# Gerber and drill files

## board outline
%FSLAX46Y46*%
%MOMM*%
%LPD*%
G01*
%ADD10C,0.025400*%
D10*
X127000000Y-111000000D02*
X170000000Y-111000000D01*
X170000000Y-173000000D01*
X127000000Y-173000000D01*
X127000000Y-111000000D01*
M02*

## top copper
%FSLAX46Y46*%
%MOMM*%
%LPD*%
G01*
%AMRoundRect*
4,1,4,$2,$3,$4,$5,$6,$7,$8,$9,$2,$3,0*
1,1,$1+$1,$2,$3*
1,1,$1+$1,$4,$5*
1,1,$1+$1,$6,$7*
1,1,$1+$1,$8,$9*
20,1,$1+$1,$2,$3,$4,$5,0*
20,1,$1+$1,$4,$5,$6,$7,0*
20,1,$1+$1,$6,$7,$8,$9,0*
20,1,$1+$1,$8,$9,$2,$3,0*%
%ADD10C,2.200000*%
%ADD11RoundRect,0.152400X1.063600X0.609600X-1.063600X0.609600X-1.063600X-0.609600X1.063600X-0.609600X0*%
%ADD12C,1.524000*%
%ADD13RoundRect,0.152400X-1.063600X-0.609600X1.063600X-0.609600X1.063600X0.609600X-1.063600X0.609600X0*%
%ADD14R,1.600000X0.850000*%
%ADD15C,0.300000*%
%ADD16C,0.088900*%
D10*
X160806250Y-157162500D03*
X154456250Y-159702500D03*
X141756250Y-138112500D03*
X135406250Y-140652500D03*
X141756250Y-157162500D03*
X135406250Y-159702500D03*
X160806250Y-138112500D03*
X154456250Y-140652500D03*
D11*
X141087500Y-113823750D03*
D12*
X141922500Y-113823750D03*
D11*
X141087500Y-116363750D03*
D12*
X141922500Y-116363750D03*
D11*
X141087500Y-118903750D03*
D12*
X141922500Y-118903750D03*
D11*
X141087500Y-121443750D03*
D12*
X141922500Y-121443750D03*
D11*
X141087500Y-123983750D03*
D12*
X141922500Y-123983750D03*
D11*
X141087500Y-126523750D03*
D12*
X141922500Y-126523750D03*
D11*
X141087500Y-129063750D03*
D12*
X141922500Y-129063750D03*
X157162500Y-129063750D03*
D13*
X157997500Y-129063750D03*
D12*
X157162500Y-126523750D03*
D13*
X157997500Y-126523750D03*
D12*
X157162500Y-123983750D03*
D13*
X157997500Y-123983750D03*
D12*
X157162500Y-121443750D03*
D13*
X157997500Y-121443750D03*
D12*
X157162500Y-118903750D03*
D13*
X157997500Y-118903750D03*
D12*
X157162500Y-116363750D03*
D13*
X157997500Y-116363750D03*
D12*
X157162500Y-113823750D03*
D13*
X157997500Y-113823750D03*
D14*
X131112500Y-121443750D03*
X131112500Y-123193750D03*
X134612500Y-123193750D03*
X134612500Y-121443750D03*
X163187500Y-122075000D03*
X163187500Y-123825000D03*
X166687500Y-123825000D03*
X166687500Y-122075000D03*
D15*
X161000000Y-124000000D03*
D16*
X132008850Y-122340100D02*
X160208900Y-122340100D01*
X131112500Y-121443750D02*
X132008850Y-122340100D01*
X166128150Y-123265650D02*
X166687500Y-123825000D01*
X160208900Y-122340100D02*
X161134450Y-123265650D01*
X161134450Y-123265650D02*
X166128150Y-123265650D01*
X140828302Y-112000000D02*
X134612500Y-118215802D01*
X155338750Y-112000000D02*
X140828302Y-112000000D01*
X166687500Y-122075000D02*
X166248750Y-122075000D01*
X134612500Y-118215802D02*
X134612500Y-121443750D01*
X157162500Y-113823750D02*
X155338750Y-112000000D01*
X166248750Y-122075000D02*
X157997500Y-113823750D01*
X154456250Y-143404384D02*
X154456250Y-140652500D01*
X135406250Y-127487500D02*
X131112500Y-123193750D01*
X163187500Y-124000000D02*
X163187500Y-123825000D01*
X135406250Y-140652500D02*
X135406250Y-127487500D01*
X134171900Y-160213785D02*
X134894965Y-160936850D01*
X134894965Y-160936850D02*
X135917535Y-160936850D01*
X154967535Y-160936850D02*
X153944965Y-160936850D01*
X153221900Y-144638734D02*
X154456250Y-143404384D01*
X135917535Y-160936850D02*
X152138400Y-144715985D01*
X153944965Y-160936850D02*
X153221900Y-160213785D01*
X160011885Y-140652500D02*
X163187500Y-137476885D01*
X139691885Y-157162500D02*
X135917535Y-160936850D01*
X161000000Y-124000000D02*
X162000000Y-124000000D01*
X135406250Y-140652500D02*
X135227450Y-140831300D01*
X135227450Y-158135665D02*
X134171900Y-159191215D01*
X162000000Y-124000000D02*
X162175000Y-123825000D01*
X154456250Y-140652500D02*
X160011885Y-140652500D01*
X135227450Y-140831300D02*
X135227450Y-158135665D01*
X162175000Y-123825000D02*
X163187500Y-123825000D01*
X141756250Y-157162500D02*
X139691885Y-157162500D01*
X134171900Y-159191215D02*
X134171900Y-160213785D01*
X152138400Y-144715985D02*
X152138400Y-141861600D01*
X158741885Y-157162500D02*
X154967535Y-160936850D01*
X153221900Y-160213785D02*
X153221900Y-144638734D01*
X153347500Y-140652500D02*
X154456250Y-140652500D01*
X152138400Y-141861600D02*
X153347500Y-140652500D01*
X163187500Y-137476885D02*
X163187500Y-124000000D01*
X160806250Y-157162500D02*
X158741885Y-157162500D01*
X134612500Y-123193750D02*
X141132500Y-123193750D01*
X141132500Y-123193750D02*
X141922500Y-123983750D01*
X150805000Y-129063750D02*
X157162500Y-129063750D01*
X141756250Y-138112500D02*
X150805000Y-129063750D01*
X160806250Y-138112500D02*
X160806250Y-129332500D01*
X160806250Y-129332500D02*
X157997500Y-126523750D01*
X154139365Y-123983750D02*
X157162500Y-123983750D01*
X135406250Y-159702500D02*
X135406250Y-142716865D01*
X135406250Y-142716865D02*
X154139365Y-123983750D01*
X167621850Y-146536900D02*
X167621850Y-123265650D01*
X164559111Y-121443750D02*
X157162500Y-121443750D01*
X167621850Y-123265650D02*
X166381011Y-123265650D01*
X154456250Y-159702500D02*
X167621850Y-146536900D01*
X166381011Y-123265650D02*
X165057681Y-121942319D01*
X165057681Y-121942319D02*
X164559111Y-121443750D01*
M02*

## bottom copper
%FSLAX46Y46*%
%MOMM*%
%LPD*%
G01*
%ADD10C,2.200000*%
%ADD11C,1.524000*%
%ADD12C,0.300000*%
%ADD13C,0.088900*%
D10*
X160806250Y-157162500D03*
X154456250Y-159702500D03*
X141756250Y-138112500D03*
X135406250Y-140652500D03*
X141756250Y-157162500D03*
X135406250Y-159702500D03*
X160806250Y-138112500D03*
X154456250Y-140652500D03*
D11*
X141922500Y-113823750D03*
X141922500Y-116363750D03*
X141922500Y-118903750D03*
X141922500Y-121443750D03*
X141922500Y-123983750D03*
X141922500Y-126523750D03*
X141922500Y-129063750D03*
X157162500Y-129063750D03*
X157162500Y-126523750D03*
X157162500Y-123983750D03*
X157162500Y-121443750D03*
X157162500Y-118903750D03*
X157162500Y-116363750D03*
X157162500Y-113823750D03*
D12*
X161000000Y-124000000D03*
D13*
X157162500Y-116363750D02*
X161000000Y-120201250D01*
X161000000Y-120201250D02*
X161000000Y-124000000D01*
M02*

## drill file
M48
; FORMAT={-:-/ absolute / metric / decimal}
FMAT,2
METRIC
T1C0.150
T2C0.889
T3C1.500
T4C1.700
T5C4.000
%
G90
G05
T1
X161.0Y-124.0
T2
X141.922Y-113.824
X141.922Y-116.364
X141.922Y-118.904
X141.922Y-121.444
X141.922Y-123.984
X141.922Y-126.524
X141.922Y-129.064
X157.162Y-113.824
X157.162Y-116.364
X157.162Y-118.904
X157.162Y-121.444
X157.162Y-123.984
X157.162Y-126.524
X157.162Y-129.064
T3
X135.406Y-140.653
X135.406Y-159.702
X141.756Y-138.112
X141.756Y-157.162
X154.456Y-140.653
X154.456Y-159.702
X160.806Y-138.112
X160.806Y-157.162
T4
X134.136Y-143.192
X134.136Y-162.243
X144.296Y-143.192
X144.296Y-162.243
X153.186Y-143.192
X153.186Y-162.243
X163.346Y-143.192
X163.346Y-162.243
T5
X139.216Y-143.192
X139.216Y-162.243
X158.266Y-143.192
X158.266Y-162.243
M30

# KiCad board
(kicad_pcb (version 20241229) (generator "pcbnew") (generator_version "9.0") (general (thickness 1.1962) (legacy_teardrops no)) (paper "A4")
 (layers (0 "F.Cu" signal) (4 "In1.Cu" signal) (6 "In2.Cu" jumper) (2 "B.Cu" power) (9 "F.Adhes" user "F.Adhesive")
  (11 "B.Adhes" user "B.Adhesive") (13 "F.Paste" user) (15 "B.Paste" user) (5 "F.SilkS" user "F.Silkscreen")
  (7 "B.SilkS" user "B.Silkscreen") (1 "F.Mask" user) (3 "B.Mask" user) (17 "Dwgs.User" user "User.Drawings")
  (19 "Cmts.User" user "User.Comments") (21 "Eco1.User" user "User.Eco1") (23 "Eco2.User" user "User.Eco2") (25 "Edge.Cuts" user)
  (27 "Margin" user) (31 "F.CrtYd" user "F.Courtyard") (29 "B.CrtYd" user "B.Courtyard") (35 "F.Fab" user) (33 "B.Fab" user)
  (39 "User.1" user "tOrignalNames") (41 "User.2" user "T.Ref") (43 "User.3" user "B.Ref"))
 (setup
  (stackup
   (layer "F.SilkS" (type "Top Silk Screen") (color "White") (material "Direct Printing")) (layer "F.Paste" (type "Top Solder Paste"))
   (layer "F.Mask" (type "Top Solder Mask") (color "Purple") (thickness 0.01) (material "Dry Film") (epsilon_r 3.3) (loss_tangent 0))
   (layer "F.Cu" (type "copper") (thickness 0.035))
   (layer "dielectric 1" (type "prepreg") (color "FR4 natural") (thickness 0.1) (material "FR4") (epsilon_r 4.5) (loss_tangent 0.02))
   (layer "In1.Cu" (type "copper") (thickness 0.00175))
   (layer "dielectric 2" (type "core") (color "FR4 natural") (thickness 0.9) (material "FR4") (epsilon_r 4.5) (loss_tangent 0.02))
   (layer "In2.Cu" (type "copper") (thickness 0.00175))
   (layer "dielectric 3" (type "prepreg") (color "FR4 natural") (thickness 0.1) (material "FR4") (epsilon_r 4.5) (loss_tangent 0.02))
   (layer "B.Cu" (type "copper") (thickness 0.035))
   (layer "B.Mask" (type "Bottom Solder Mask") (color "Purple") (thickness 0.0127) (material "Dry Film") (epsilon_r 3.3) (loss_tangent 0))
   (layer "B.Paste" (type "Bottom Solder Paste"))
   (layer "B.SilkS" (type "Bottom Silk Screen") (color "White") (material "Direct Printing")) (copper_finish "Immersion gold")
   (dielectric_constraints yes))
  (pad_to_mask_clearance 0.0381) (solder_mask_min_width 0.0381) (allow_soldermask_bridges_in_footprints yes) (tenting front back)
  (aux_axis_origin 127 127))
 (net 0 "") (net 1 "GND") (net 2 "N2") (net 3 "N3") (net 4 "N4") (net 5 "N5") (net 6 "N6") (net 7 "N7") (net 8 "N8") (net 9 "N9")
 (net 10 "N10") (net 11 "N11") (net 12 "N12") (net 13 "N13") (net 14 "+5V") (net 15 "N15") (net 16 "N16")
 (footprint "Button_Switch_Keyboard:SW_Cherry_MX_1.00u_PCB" (layer "F.Cu") (at 160.80625 157.1625)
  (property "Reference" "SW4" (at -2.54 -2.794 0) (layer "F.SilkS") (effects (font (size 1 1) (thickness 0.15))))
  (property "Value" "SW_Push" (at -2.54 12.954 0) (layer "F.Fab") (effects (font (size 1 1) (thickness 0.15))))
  (pad "" np_thru_hole circle (at -7.62 5.08) (size 1.7 1.7) (drill 1.7) (layers "*.Cu" "*.Mask"))
  (pad "" np_thru_hole circle (at -2.54 5.08) (size 4 4) (drill 4) (layers "*.Cu" "*.Mask"))
  (pad "" np_thru_hole circle (at 2.54 5.08) (size 1.7 1.7) (drill 1.7) (layers "*.Cu" "*.Mask"))
  (pad "1" thru_hole circle (at 0 0) (size 2.2 2.2) (drill 1.5) (layers "*.Cu" "*.Mask") (remove_unused_layers no) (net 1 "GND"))
  (pad "2" thru_hole circle (at -6.35 2.54) (size 2.2 2.2) (drill 1.5) (layers "*.Cu" "*.Mask") (remove_unused_layers no) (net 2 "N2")))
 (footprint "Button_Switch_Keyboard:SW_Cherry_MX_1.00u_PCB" (layer "F.Cu") (at 141.75625 138.1125)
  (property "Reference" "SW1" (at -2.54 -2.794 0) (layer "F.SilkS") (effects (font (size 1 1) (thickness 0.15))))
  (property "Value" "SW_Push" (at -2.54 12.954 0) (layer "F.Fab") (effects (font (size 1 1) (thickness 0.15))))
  (pad "" np_thru_hole circle (at -7.62 5.08) (size 1.7 1.7) (drill 1.7) (layers "*.Cu" "*.Mask"))
  (pad "" np_thru_hole circle (at -2.54 5.08) (size 4 4) (drill 4) (layers "*.Cu" "*.Mask"))
  (pad "" np_thru_hole circle (at 2.54 5.08) (size 1.7 1.7) (drill 1.7) (layers "*.Cu" "*.Mask"))
  (pad "1" thru_hole circle (at 0 0) (size 2.2 2.2) (drill 1.5) (layers "*.Cu" "*.Mask") (remove_unused_layers no) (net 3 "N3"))
  (pad "2" thru_hole circle (at -6.35 2.54) (size 2.2 2.2) (drill 1.5) (layers "*.Cu" "*.Mask") (remove_unused_layers no) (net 1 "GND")))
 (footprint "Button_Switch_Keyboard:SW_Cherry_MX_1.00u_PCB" (layer "F.Cu") (at 141.75625 157.1625)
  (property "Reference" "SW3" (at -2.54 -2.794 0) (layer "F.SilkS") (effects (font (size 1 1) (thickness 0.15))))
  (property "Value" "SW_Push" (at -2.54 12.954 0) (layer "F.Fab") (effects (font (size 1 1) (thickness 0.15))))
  (pad "" np_thru_hole circle (at -7.62 5.08) (size 1.7 1.7) (drill 1.7) (layers "*.Cu" "*.Mask"))
  (pad "" np_thru_hole circle (at -2.54 5.08) (size 4 4) (drill 4) (layers "*.Cu" "*.Mask"))
  (pad "" np_thru_hole circle (at 2.54 5.08) (size 1.7 1.7) (drill 1.7) (layers "*.Cu" "*.Mask"))
  (pad "1" thru_hole circle (at 0 0) (size 2.2 2.2) (drill 1.5) (layers "*.Cu" "*.Mask") (remove_unused_layers no) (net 1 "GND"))
  (pad "2" thru_hole circle (at -6.35 2.54) (size 2.2 2.2) (drill 1.5) (layers "*.Cu" "*.Mask") (remove_unused_layers no) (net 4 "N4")))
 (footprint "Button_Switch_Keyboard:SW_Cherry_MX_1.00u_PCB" (layer "F.Cu") (at 160.80625 138.1125)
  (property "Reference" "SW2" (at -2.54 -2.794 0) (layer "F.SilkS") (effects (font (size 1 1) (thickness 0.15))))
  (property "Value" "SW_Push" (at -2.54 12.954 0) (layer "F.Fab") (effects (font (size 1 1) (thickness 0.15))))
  (pad "" np_thru_hole circle (at -7.62 5.08) (size 1.7 1.7) (drill 1.7) (layers "*.Cu" "*.Mask"))
  (pad "" np_thru_hole circle (at -2.54 5.08) (size 4 4) (drill 4) (layers "*.Cu" "*.Mask"))
  (pad "" np_thru_hole circle (at 2.54 5.08) (size 1.7 1.7) (drill 1.7) (layers "*.Cu" "*.Mask"))
  (pad "1" thru_hole circle (at 0 0) (size 2.2 2.2) (drill 1.5) (layers "*.Cu" "*.Mask") (remove_unused_layers no) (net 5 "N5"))
  (pad "2" thru_hole circle (at -6.35 2.54) (size 2.2 2.2) (drill 1.5) (layers "*.Cu" "*.Mask") (remove_unused_layers no) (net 1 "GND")))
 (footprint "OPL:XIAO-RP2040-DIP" (layer "F.Cu") (at 149.5425 121.44375)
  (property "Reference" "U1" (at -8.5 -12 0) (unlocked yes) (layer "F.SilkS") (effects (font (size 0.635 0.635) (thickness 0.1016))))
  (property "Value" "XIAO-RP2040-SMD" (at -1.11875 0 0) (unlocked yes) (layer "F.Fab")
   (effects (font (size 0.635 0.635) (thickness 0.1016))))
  (pad "1" smd roundrect (at -8.455 -7.62 180) (size 2.432 1.524) (layers "F.Cu" "F.Mask") (roundrect_rratio 0.1) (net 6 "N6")
   (thermal_bridge_angle 45))
  (pad "1" thru_hole circle (at -7.62 -7.62 180) (size 1.524 1.524) (drill 0.889) (layers "*.Cu" "*.Mask") (remove_unused_layers no)
   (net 6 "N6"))
  (pad "2" smd roundrect (at -8.455 -5.08 180) (size 2.432 1.524) (layers "F.Cu" "F.Mask") (roundrect_rratio 0.1) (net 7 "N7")
   (thermal_bridge_angle 45))
  (pad "2" thru_hole circle (at -7.62 -5.08 180) (size 1.524 1.524) (drill 0.889) (layers "*.Cu" "*.Mask") (remove_unused_layers no)
   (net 7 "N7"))
  (pad "3" smd roundrect (at -8.455 -2.54 180) (size 2.432 1.524) (layers "F.Cu" "F.Mask") (roundrect_rratio 0.1) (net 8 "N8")
   (thermal_bridge_angle 45))
  (pad "3" thru_hole circle (at -7.62 -2.54 180) (size 1.524 1.524) (drill 0.889) (layers "*.Cu" "*.Mask") (remove_unused_layers no)
   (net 8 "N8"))
  (pad "4" smd roundrect (at -8.455 0 180) (size 2.432 1.524) (layers "F.Cu" "F.Mask") (roundrect_rratio 0.1) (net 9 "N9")
   (thermal_bridge_angle 45))
  (pad "4" thru_hole circle (at -7.62 0 180) (size 1.524 1.524) (drill 0.889) (layers "*.Cu" "*.Mask") (remove_unused_layers no)
   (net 9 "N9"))
  (pad "5" smd roundrect (at -8.455 2.54 180) (size 2.432 1.524) (layers "F.Cu" "F.Mask") (roundrect_rratio 0.1) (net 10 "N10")
   (thermal_bridge_angle 45))
  (pad "5" thru_hole circle (at -7.62 2.54 180) (size 1.524 1.524) (drill 0.889) (layers "*.Cu" "*.Mask") (remove_unused_layers no)
   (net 10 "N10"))
  (pad "6" smd roundrect (at -8.455 5.08 180) (size 2.432 1.524) (layers "F.Cu" "F.Mask") (roundrect_rratio 0.1) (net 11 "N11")
   (thermal_bridge_angle 45))
  (pad "6" thru_hole circle (at -7.62 5.08 180) (size 1.524 1.524) (drill 0.889) (layers "*.Cu" "*.Mask") (remove_unused_layers no)
   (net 11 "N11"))
  (pad "7" smd roundrect (at -8.455 7.62 180) (size 2.432 1.524) (layers "F.Cu" "F.Mask") (roundrect_rratio 0.1) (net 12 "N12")
   (thermal_bridge_angle 45))
  (pad "7" thru_hole circle (at -7.62 7.62 180) (size 1.524 1.524) (drill 0.889) (layers "*.Cu" "*.Mask") (remove_unused_layers no)
   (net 12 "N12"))
  (pad "8" thru_hole circle (at 7.62 7.62) (size 1.524 1.524) (drill 0.889) (layers "*.Cu" "*.Mask") (remove_unused_layers no) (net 3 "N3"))
  (pad "8" smd roundrect (at 8.455 7.62) (size 2.432 1.524) (layers "F.Cu" "F.Mask") (roundrect_rratio 0.1) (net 3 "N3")
   (thermal_bridge_angle 45))
  (pad "9" thru_hole circle (at 7.62 5.08) (size 1.524 1.524) (drill 0.889) (layers "*.Cu" "*.Mask") (remove_unused_layers no) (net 5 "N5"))
  (pad "9" smd roundrect (at 8.455 5.08) (size 2.432 1.524) (layers "F.Cu" "F.Mask") (roundrect_rratio 0.1) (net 5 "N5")
   (thermal_bridge_angle 45))
  (pad "10" thru_hole circle (at 7.62 2.54) (size 1.524 1.524) (drill 0.889) (layers "*.Cu" "*.Mask") (remove_unused_layers no) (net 4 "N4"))
  (pad "10" smd roundrect (at 8.455 2.54) (size 2.432 1.524) (layers "F.Cu" "F.Mask") (roundrect_rratio 0.1) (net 4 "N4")
   (thermal_bridge_angle 45))
  (pad "11" thru_hole circle (at 7.62 0) (size 1.524 1.524) (drill 0.889) (layers "*.Cu" "*.Mask") (remove_unused_layers no) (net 2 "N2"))
  (pad "11" smd roundrect (at 8.455 0) (size 2.432 1.524) (layers "F.Cu" "F.Mask") (roundrect_rratio 0.1) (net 2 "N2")
   (thermal_bridge_angle 45))
  (pad "12" thru_hole circle (at 7.62 -2.54) (size 1.524 1.524) (drill 0.889) (layers "*.Cu" "*.Mask") (remove_unused_layers no)
   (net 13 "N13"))
  (pad "12" smd roundrect (at 8.455 -2.54) (size 2.432 1.524) (layers "F.Cu" "F.Mask") (roundrect_rratio 0.1) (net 13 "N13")
   (thermal_bridge_angle 45))
  (pad "13" thru_hole circle (at 7.62 -5.08) (size 1.524 1.524) (drill 0.889) (layers "*.Cu" "*.Mask") (remove_unused_layers no)
   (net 1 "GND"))
  (pad "13" smd roundrect (at 8.455 -5.08) (size 2.432 1.524) (layers "F.Cu" "F.Mask") (roundrect_rratio 0.1) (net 1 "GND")
   (thermal_bridge_angle 45))
  (pad "14" thru_hole circle (at 7.62 -7.62) (size 1.524 1.524) (drill 0.889) (layers "*.Cu" "*.Mask") (remove_unused_layers no)
   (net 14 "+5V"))
  (pad "14" smd roundrect (at 8.455 -7.62) (size 2.432 1.524) (layers "F.Cu" "F.Mask") (roundrect_rratio 0.1) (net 14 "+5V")
   (thermal_bridge_angle 45)))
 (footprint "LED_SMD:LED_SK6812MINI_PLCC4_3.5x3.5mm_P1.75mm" (layer "F.Cu") (at 132.8625 122.31875)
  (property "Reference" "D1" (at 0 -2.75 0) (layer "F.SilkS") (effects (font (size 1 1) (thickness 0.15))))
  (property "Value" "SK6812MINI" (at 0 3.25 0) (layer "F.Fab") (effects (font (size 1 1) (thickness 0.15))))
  (pad "1" smd rect (at -1.75 -0.875) (size 1.6 0.85) (layers "F.Cu" "F.Mask" "F.Paste") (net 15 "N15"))
  (pad "2" smd rect (at -1.75 0.875) (size 1.6 0.85) (layers "F.Cu" "F.Mask" "F.Paste") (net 1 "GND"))
  (pad "3" smd rect (at 1.75 0.875) (size 1.6 0.85) (layers "F.Cu" "F.Mask" "F.Paste") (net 10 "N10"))
  (pad "4" smd rect (at 1.75 -0.875) (size 1.6 0.85) (layers "F.Cu" "F.Mask" "F.Paste") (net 14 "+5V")))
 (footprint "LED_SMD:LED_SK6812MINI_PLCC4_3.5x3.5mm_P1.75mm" (layer "F.Cu") (at 164.9375 122.95)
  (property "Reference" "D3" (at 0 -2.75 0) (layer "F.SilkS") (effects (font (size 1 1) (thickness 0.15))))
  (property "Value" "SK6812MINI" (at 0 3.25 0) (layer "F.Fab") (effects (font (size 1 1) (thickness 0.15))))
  (pad "1" smd rect (at -1.75 -0.875) (size 1.6 0.85) (layers "F.Cu" "F.Mask" "F.Paste") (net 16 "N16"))
  (pad "2" smd rect (at -1.75 0.875) (size 1.6 0.85) (layers "F.Cu" "F.Mask" "F.Paste") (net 1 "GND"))
  (pad "3" smd rect (at 1.75 0.875) (size 1.6 0.85) (layers "F.Cu" "F.Mask" "F.Paste") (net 15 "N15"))
  (pad "4" smd rect (at 1.75 -0.875) (size 1.6 0.85) (layers "F.Cu" "F.Mask" "F.Paste") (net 14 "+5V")))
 (gr_rect (start 127 111) (end 170 173) (stroke (width 0.0254) (type default)) (fill no) (layer "Edge.Cuts"))
 (segment (start 132.00885 122.3401) (end 160.2089 122.3401) (width 0.0889) (layer "F.Cu") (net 15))
 (segment (start 131.1125 121.44375) (end 132.00885 122.3401) (width 0.0889) (layer "F.Cu") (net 15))
 (segment (start 166.12815 123.26565) (end 166.6875 123.825) (width 0.0889) (layer "F.Cu") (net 15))
 (segment (start 160.2089 122.3401) (end 161.13445 123.26565) (width 0.0889) (layer "F.Cu") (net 15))
 (segment (start 161.13445 123.26565) (end 166.12815 123.26565) (width 0.0889) (layer "F.Cu") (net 15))
 (segment (start 140.828302 112) (end 134.6125 118.215802) (width 0.0889) (layer "F.Cu") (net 14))
 (segment (start 155.33875 112) (end 140.828302 112) (width 0.0889) (layer "F.Cu") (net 14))
 (segment (start 166.6875 122.075) (end 166.24875 122.075) (width 0.0889) (layer "F.Cu") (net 14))
 (segment (start 134.6125 118.215802) (end 134.6125 121.44375) (width 0.0889) (layer "F.Cu") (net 14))
 (segment (start 157.1625 113.82375) (end 155.33875 112) (width 0.0889) (layer "F.Cu") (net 14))
 (segment (start 166.24875 122.075) (end 157.9975 113.82375) (width 0.0889) (layer "F.Cu") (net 14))
 (segment (start 154.45625 143.404384) (end 154.45625 140.6525) (width 0.0889) (layer "F.Cu") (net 1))
 (segment (start 135.40625 127.4875) (end 131.1125 123.19375) (width 0.0889) (layer "F.Cu") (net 1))
 (segment (start 163.1875 124) (end 163.1875 123.825) (width 0.0889) (layer "F.Cu") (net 1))
 (segment (start 135.40625 140.6525) (end 135.40625 127.4875) (width 0.0889) (layer "F.Cu") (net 1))
 (segment (start 134.1719 160.213785) (end 134.894965 160.93685) (width 0.0889) (layer "F.Cu") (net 1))
 (segment (start 134.894965 160.93685) (end 135.917535 160.93685) (width 0.0889) (layer "F.Cu") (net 1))
 (segment (start 154.967535 160.93685) (end 153.944965 160.93685) (width 0.0889) (layer "F.Cu") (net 1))
 (segment (start 153.2219 144.638734) (end 154.45625 143.404384) (width 0.0889) (layer "F.Cu") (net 1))
 (segment (start 135.917535 160.93685) (end 152.1384 144.715985) (width 0.0889) (layer "F.Cu") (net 1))
 (segment (start 153.944965 160.93685) (end 153.2219 160.213785) (width 0.0889) (layer "F.Cu") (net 1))
 (segment (start 160.011885 140.6525) (end 163.1875 137.476885) (width 0.0889) (layer "F.Cu") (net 1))
 (segment (start 139.691885 157.1625) (end 135.917535 160.93685) (width 0.0889) (layer "F.Cu") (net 1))
 (segment (start 161 124) (end 162 124) (width 0.0889) (layer "F.Cu") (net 1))
 (segment (start 135.40625 140.6525) (end 135.22745 140.8313) (width 0.0889) (layer "F.Cu") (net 1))
 (segment (start 135.22745 158.135665) (end 134.1719 159.191215) (width 0.0889) (layer "F.Cu") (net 1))
 (segment (start 162 124) (end 162.175 123.825) (width 0.0889) (layer "F.Cu") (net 1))
 (segment (start 154.45625 140.6525) (end 160.011885 140.6525) (width 0.0889) (layer "F.Cu") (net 1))
 (segment (start 135.22745 140.8313) (end 135.22745 158.135665) (width 0.0889) (layer "F.Cu") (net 1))
 (segment (start 162.175 123.825) (end 163.1875 123.825) (width 0.0889) (layer "F.Cu") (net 1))
 (segment (start 141.75625 157.1625) (end 139.691885 157.1625) (width 0.0889) (layer "F.Cu") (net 1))
 (segment (start 134.1719 159.191215) (end 134.1719 160.213785) (width 0.0889) (layer "F.Cu") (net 1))
 (segment (start 152.1384 144.715985) (end 152.1384 141.8616) (width 0.0889) (layer "F.Cu") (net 1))
 (segment (start 158.741885 157.1625) (end 154.967535 160.93685) (width 0.0889) (layer "F.Cu") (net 1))
 (segment (start 153.2219 160.213785) (end 153.2219 144.638734) (width 0.0889) (layer "F.Cu") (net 1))
 (segment (start 153.3475 140.6525) (end 154.45625 140.6525) (width 0.0889) (layer "F.Cu") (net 1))
 (segment (start 152.1384 141.8616) (end 153.3475 140.6525) (width 0.0889) (layer "F.Cu") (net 1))
 (segment (start 163.1875 137.476885) (end 163.1875 124) (width 0.0889) (layer "F.Cu") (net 1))
 (segment (start 160.80625 157.1625) (end 158.741885 157.1625) (width 0.0889) (layer "F.Cu") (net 1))
 (via (at 161 124) (size 0.3) (drill 0.15) (layers "F.Cu" "B.Cu") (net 1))
 (segment (start 157.1625 116.36375) (end 161 120.20125) (width 0.0889) (layer "B.Cu") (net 1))
 (segment (start 161 120.20125) (end 161 124) (width 0.0889) (layer "B.Cu") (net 1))
 (segment (start 134.6125 123.19375) (end 141.1325 123.19375) (width 0.0889) (layer "F.Cu") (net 10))
 (segment (start 141.1325 123.19375) (end 141.9225 123.98375) (width 0.0889) (layer "F.Cu") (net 10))
 (segment (start 150.805 129.06375) (end 157.1625 129.06375) (width 0.0889) (layer "F.Cu") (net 3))
 (segment (start 141.75625 138.1125) (end 150.805 129.06375) (width 0.0889) (layer "F.Cu") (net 3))
 (segment (start 160.80625 138.1125) (end 160.80625 129.3325) (width 0.0889) (layer "F.Cu") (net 5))
 (segment (start 160.80625 129.3325) (end 157.9975 126.52375) (width 0.0889) (layer "F.Cu") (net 5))
 (segment (start 154.139365 123.98375) (end 157.1625 123.98375) (width 0.0889) (layer "F.Cu") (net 4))
 (segment (start 135.40625 159.7025) (end 135.40625 142.716865) (width 0.0889) (layer "F.Cu") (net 4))
 (segment (start 135.40625 142.716865) (end 154.139365 123.98375) (width 0.0889) (layer "F.Cu") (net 4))
 (segment (start 167.62185 146.5369) (end 167.62185 123.26565) (width 0.0889) (layer "F.Cu") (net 2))
 (segment (start 164.559111 121.44375) (end 157.1625 121.44375) (width 0.0889) (layer "F.Cu") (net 2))
 (segment (start 167.62185 123.26565) (end 166.381011 123.26565) (width 0.0889) (layer "F.Cu") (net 2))
 (segment (start 154.45625 159.7025) (end 167.62185 146.5369) (width 0.0889) (layer "F.Cu") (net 2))
 (segment (start 166.381011 123.26565) (end 165.057681 121.942319) (width 0.0889) (layer "F.Cu") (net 2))
 (segment (start 165.057681 121.942319) (end 164.559111 121.44375) (width 0.0889) (layer "F.Cu") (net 2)))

